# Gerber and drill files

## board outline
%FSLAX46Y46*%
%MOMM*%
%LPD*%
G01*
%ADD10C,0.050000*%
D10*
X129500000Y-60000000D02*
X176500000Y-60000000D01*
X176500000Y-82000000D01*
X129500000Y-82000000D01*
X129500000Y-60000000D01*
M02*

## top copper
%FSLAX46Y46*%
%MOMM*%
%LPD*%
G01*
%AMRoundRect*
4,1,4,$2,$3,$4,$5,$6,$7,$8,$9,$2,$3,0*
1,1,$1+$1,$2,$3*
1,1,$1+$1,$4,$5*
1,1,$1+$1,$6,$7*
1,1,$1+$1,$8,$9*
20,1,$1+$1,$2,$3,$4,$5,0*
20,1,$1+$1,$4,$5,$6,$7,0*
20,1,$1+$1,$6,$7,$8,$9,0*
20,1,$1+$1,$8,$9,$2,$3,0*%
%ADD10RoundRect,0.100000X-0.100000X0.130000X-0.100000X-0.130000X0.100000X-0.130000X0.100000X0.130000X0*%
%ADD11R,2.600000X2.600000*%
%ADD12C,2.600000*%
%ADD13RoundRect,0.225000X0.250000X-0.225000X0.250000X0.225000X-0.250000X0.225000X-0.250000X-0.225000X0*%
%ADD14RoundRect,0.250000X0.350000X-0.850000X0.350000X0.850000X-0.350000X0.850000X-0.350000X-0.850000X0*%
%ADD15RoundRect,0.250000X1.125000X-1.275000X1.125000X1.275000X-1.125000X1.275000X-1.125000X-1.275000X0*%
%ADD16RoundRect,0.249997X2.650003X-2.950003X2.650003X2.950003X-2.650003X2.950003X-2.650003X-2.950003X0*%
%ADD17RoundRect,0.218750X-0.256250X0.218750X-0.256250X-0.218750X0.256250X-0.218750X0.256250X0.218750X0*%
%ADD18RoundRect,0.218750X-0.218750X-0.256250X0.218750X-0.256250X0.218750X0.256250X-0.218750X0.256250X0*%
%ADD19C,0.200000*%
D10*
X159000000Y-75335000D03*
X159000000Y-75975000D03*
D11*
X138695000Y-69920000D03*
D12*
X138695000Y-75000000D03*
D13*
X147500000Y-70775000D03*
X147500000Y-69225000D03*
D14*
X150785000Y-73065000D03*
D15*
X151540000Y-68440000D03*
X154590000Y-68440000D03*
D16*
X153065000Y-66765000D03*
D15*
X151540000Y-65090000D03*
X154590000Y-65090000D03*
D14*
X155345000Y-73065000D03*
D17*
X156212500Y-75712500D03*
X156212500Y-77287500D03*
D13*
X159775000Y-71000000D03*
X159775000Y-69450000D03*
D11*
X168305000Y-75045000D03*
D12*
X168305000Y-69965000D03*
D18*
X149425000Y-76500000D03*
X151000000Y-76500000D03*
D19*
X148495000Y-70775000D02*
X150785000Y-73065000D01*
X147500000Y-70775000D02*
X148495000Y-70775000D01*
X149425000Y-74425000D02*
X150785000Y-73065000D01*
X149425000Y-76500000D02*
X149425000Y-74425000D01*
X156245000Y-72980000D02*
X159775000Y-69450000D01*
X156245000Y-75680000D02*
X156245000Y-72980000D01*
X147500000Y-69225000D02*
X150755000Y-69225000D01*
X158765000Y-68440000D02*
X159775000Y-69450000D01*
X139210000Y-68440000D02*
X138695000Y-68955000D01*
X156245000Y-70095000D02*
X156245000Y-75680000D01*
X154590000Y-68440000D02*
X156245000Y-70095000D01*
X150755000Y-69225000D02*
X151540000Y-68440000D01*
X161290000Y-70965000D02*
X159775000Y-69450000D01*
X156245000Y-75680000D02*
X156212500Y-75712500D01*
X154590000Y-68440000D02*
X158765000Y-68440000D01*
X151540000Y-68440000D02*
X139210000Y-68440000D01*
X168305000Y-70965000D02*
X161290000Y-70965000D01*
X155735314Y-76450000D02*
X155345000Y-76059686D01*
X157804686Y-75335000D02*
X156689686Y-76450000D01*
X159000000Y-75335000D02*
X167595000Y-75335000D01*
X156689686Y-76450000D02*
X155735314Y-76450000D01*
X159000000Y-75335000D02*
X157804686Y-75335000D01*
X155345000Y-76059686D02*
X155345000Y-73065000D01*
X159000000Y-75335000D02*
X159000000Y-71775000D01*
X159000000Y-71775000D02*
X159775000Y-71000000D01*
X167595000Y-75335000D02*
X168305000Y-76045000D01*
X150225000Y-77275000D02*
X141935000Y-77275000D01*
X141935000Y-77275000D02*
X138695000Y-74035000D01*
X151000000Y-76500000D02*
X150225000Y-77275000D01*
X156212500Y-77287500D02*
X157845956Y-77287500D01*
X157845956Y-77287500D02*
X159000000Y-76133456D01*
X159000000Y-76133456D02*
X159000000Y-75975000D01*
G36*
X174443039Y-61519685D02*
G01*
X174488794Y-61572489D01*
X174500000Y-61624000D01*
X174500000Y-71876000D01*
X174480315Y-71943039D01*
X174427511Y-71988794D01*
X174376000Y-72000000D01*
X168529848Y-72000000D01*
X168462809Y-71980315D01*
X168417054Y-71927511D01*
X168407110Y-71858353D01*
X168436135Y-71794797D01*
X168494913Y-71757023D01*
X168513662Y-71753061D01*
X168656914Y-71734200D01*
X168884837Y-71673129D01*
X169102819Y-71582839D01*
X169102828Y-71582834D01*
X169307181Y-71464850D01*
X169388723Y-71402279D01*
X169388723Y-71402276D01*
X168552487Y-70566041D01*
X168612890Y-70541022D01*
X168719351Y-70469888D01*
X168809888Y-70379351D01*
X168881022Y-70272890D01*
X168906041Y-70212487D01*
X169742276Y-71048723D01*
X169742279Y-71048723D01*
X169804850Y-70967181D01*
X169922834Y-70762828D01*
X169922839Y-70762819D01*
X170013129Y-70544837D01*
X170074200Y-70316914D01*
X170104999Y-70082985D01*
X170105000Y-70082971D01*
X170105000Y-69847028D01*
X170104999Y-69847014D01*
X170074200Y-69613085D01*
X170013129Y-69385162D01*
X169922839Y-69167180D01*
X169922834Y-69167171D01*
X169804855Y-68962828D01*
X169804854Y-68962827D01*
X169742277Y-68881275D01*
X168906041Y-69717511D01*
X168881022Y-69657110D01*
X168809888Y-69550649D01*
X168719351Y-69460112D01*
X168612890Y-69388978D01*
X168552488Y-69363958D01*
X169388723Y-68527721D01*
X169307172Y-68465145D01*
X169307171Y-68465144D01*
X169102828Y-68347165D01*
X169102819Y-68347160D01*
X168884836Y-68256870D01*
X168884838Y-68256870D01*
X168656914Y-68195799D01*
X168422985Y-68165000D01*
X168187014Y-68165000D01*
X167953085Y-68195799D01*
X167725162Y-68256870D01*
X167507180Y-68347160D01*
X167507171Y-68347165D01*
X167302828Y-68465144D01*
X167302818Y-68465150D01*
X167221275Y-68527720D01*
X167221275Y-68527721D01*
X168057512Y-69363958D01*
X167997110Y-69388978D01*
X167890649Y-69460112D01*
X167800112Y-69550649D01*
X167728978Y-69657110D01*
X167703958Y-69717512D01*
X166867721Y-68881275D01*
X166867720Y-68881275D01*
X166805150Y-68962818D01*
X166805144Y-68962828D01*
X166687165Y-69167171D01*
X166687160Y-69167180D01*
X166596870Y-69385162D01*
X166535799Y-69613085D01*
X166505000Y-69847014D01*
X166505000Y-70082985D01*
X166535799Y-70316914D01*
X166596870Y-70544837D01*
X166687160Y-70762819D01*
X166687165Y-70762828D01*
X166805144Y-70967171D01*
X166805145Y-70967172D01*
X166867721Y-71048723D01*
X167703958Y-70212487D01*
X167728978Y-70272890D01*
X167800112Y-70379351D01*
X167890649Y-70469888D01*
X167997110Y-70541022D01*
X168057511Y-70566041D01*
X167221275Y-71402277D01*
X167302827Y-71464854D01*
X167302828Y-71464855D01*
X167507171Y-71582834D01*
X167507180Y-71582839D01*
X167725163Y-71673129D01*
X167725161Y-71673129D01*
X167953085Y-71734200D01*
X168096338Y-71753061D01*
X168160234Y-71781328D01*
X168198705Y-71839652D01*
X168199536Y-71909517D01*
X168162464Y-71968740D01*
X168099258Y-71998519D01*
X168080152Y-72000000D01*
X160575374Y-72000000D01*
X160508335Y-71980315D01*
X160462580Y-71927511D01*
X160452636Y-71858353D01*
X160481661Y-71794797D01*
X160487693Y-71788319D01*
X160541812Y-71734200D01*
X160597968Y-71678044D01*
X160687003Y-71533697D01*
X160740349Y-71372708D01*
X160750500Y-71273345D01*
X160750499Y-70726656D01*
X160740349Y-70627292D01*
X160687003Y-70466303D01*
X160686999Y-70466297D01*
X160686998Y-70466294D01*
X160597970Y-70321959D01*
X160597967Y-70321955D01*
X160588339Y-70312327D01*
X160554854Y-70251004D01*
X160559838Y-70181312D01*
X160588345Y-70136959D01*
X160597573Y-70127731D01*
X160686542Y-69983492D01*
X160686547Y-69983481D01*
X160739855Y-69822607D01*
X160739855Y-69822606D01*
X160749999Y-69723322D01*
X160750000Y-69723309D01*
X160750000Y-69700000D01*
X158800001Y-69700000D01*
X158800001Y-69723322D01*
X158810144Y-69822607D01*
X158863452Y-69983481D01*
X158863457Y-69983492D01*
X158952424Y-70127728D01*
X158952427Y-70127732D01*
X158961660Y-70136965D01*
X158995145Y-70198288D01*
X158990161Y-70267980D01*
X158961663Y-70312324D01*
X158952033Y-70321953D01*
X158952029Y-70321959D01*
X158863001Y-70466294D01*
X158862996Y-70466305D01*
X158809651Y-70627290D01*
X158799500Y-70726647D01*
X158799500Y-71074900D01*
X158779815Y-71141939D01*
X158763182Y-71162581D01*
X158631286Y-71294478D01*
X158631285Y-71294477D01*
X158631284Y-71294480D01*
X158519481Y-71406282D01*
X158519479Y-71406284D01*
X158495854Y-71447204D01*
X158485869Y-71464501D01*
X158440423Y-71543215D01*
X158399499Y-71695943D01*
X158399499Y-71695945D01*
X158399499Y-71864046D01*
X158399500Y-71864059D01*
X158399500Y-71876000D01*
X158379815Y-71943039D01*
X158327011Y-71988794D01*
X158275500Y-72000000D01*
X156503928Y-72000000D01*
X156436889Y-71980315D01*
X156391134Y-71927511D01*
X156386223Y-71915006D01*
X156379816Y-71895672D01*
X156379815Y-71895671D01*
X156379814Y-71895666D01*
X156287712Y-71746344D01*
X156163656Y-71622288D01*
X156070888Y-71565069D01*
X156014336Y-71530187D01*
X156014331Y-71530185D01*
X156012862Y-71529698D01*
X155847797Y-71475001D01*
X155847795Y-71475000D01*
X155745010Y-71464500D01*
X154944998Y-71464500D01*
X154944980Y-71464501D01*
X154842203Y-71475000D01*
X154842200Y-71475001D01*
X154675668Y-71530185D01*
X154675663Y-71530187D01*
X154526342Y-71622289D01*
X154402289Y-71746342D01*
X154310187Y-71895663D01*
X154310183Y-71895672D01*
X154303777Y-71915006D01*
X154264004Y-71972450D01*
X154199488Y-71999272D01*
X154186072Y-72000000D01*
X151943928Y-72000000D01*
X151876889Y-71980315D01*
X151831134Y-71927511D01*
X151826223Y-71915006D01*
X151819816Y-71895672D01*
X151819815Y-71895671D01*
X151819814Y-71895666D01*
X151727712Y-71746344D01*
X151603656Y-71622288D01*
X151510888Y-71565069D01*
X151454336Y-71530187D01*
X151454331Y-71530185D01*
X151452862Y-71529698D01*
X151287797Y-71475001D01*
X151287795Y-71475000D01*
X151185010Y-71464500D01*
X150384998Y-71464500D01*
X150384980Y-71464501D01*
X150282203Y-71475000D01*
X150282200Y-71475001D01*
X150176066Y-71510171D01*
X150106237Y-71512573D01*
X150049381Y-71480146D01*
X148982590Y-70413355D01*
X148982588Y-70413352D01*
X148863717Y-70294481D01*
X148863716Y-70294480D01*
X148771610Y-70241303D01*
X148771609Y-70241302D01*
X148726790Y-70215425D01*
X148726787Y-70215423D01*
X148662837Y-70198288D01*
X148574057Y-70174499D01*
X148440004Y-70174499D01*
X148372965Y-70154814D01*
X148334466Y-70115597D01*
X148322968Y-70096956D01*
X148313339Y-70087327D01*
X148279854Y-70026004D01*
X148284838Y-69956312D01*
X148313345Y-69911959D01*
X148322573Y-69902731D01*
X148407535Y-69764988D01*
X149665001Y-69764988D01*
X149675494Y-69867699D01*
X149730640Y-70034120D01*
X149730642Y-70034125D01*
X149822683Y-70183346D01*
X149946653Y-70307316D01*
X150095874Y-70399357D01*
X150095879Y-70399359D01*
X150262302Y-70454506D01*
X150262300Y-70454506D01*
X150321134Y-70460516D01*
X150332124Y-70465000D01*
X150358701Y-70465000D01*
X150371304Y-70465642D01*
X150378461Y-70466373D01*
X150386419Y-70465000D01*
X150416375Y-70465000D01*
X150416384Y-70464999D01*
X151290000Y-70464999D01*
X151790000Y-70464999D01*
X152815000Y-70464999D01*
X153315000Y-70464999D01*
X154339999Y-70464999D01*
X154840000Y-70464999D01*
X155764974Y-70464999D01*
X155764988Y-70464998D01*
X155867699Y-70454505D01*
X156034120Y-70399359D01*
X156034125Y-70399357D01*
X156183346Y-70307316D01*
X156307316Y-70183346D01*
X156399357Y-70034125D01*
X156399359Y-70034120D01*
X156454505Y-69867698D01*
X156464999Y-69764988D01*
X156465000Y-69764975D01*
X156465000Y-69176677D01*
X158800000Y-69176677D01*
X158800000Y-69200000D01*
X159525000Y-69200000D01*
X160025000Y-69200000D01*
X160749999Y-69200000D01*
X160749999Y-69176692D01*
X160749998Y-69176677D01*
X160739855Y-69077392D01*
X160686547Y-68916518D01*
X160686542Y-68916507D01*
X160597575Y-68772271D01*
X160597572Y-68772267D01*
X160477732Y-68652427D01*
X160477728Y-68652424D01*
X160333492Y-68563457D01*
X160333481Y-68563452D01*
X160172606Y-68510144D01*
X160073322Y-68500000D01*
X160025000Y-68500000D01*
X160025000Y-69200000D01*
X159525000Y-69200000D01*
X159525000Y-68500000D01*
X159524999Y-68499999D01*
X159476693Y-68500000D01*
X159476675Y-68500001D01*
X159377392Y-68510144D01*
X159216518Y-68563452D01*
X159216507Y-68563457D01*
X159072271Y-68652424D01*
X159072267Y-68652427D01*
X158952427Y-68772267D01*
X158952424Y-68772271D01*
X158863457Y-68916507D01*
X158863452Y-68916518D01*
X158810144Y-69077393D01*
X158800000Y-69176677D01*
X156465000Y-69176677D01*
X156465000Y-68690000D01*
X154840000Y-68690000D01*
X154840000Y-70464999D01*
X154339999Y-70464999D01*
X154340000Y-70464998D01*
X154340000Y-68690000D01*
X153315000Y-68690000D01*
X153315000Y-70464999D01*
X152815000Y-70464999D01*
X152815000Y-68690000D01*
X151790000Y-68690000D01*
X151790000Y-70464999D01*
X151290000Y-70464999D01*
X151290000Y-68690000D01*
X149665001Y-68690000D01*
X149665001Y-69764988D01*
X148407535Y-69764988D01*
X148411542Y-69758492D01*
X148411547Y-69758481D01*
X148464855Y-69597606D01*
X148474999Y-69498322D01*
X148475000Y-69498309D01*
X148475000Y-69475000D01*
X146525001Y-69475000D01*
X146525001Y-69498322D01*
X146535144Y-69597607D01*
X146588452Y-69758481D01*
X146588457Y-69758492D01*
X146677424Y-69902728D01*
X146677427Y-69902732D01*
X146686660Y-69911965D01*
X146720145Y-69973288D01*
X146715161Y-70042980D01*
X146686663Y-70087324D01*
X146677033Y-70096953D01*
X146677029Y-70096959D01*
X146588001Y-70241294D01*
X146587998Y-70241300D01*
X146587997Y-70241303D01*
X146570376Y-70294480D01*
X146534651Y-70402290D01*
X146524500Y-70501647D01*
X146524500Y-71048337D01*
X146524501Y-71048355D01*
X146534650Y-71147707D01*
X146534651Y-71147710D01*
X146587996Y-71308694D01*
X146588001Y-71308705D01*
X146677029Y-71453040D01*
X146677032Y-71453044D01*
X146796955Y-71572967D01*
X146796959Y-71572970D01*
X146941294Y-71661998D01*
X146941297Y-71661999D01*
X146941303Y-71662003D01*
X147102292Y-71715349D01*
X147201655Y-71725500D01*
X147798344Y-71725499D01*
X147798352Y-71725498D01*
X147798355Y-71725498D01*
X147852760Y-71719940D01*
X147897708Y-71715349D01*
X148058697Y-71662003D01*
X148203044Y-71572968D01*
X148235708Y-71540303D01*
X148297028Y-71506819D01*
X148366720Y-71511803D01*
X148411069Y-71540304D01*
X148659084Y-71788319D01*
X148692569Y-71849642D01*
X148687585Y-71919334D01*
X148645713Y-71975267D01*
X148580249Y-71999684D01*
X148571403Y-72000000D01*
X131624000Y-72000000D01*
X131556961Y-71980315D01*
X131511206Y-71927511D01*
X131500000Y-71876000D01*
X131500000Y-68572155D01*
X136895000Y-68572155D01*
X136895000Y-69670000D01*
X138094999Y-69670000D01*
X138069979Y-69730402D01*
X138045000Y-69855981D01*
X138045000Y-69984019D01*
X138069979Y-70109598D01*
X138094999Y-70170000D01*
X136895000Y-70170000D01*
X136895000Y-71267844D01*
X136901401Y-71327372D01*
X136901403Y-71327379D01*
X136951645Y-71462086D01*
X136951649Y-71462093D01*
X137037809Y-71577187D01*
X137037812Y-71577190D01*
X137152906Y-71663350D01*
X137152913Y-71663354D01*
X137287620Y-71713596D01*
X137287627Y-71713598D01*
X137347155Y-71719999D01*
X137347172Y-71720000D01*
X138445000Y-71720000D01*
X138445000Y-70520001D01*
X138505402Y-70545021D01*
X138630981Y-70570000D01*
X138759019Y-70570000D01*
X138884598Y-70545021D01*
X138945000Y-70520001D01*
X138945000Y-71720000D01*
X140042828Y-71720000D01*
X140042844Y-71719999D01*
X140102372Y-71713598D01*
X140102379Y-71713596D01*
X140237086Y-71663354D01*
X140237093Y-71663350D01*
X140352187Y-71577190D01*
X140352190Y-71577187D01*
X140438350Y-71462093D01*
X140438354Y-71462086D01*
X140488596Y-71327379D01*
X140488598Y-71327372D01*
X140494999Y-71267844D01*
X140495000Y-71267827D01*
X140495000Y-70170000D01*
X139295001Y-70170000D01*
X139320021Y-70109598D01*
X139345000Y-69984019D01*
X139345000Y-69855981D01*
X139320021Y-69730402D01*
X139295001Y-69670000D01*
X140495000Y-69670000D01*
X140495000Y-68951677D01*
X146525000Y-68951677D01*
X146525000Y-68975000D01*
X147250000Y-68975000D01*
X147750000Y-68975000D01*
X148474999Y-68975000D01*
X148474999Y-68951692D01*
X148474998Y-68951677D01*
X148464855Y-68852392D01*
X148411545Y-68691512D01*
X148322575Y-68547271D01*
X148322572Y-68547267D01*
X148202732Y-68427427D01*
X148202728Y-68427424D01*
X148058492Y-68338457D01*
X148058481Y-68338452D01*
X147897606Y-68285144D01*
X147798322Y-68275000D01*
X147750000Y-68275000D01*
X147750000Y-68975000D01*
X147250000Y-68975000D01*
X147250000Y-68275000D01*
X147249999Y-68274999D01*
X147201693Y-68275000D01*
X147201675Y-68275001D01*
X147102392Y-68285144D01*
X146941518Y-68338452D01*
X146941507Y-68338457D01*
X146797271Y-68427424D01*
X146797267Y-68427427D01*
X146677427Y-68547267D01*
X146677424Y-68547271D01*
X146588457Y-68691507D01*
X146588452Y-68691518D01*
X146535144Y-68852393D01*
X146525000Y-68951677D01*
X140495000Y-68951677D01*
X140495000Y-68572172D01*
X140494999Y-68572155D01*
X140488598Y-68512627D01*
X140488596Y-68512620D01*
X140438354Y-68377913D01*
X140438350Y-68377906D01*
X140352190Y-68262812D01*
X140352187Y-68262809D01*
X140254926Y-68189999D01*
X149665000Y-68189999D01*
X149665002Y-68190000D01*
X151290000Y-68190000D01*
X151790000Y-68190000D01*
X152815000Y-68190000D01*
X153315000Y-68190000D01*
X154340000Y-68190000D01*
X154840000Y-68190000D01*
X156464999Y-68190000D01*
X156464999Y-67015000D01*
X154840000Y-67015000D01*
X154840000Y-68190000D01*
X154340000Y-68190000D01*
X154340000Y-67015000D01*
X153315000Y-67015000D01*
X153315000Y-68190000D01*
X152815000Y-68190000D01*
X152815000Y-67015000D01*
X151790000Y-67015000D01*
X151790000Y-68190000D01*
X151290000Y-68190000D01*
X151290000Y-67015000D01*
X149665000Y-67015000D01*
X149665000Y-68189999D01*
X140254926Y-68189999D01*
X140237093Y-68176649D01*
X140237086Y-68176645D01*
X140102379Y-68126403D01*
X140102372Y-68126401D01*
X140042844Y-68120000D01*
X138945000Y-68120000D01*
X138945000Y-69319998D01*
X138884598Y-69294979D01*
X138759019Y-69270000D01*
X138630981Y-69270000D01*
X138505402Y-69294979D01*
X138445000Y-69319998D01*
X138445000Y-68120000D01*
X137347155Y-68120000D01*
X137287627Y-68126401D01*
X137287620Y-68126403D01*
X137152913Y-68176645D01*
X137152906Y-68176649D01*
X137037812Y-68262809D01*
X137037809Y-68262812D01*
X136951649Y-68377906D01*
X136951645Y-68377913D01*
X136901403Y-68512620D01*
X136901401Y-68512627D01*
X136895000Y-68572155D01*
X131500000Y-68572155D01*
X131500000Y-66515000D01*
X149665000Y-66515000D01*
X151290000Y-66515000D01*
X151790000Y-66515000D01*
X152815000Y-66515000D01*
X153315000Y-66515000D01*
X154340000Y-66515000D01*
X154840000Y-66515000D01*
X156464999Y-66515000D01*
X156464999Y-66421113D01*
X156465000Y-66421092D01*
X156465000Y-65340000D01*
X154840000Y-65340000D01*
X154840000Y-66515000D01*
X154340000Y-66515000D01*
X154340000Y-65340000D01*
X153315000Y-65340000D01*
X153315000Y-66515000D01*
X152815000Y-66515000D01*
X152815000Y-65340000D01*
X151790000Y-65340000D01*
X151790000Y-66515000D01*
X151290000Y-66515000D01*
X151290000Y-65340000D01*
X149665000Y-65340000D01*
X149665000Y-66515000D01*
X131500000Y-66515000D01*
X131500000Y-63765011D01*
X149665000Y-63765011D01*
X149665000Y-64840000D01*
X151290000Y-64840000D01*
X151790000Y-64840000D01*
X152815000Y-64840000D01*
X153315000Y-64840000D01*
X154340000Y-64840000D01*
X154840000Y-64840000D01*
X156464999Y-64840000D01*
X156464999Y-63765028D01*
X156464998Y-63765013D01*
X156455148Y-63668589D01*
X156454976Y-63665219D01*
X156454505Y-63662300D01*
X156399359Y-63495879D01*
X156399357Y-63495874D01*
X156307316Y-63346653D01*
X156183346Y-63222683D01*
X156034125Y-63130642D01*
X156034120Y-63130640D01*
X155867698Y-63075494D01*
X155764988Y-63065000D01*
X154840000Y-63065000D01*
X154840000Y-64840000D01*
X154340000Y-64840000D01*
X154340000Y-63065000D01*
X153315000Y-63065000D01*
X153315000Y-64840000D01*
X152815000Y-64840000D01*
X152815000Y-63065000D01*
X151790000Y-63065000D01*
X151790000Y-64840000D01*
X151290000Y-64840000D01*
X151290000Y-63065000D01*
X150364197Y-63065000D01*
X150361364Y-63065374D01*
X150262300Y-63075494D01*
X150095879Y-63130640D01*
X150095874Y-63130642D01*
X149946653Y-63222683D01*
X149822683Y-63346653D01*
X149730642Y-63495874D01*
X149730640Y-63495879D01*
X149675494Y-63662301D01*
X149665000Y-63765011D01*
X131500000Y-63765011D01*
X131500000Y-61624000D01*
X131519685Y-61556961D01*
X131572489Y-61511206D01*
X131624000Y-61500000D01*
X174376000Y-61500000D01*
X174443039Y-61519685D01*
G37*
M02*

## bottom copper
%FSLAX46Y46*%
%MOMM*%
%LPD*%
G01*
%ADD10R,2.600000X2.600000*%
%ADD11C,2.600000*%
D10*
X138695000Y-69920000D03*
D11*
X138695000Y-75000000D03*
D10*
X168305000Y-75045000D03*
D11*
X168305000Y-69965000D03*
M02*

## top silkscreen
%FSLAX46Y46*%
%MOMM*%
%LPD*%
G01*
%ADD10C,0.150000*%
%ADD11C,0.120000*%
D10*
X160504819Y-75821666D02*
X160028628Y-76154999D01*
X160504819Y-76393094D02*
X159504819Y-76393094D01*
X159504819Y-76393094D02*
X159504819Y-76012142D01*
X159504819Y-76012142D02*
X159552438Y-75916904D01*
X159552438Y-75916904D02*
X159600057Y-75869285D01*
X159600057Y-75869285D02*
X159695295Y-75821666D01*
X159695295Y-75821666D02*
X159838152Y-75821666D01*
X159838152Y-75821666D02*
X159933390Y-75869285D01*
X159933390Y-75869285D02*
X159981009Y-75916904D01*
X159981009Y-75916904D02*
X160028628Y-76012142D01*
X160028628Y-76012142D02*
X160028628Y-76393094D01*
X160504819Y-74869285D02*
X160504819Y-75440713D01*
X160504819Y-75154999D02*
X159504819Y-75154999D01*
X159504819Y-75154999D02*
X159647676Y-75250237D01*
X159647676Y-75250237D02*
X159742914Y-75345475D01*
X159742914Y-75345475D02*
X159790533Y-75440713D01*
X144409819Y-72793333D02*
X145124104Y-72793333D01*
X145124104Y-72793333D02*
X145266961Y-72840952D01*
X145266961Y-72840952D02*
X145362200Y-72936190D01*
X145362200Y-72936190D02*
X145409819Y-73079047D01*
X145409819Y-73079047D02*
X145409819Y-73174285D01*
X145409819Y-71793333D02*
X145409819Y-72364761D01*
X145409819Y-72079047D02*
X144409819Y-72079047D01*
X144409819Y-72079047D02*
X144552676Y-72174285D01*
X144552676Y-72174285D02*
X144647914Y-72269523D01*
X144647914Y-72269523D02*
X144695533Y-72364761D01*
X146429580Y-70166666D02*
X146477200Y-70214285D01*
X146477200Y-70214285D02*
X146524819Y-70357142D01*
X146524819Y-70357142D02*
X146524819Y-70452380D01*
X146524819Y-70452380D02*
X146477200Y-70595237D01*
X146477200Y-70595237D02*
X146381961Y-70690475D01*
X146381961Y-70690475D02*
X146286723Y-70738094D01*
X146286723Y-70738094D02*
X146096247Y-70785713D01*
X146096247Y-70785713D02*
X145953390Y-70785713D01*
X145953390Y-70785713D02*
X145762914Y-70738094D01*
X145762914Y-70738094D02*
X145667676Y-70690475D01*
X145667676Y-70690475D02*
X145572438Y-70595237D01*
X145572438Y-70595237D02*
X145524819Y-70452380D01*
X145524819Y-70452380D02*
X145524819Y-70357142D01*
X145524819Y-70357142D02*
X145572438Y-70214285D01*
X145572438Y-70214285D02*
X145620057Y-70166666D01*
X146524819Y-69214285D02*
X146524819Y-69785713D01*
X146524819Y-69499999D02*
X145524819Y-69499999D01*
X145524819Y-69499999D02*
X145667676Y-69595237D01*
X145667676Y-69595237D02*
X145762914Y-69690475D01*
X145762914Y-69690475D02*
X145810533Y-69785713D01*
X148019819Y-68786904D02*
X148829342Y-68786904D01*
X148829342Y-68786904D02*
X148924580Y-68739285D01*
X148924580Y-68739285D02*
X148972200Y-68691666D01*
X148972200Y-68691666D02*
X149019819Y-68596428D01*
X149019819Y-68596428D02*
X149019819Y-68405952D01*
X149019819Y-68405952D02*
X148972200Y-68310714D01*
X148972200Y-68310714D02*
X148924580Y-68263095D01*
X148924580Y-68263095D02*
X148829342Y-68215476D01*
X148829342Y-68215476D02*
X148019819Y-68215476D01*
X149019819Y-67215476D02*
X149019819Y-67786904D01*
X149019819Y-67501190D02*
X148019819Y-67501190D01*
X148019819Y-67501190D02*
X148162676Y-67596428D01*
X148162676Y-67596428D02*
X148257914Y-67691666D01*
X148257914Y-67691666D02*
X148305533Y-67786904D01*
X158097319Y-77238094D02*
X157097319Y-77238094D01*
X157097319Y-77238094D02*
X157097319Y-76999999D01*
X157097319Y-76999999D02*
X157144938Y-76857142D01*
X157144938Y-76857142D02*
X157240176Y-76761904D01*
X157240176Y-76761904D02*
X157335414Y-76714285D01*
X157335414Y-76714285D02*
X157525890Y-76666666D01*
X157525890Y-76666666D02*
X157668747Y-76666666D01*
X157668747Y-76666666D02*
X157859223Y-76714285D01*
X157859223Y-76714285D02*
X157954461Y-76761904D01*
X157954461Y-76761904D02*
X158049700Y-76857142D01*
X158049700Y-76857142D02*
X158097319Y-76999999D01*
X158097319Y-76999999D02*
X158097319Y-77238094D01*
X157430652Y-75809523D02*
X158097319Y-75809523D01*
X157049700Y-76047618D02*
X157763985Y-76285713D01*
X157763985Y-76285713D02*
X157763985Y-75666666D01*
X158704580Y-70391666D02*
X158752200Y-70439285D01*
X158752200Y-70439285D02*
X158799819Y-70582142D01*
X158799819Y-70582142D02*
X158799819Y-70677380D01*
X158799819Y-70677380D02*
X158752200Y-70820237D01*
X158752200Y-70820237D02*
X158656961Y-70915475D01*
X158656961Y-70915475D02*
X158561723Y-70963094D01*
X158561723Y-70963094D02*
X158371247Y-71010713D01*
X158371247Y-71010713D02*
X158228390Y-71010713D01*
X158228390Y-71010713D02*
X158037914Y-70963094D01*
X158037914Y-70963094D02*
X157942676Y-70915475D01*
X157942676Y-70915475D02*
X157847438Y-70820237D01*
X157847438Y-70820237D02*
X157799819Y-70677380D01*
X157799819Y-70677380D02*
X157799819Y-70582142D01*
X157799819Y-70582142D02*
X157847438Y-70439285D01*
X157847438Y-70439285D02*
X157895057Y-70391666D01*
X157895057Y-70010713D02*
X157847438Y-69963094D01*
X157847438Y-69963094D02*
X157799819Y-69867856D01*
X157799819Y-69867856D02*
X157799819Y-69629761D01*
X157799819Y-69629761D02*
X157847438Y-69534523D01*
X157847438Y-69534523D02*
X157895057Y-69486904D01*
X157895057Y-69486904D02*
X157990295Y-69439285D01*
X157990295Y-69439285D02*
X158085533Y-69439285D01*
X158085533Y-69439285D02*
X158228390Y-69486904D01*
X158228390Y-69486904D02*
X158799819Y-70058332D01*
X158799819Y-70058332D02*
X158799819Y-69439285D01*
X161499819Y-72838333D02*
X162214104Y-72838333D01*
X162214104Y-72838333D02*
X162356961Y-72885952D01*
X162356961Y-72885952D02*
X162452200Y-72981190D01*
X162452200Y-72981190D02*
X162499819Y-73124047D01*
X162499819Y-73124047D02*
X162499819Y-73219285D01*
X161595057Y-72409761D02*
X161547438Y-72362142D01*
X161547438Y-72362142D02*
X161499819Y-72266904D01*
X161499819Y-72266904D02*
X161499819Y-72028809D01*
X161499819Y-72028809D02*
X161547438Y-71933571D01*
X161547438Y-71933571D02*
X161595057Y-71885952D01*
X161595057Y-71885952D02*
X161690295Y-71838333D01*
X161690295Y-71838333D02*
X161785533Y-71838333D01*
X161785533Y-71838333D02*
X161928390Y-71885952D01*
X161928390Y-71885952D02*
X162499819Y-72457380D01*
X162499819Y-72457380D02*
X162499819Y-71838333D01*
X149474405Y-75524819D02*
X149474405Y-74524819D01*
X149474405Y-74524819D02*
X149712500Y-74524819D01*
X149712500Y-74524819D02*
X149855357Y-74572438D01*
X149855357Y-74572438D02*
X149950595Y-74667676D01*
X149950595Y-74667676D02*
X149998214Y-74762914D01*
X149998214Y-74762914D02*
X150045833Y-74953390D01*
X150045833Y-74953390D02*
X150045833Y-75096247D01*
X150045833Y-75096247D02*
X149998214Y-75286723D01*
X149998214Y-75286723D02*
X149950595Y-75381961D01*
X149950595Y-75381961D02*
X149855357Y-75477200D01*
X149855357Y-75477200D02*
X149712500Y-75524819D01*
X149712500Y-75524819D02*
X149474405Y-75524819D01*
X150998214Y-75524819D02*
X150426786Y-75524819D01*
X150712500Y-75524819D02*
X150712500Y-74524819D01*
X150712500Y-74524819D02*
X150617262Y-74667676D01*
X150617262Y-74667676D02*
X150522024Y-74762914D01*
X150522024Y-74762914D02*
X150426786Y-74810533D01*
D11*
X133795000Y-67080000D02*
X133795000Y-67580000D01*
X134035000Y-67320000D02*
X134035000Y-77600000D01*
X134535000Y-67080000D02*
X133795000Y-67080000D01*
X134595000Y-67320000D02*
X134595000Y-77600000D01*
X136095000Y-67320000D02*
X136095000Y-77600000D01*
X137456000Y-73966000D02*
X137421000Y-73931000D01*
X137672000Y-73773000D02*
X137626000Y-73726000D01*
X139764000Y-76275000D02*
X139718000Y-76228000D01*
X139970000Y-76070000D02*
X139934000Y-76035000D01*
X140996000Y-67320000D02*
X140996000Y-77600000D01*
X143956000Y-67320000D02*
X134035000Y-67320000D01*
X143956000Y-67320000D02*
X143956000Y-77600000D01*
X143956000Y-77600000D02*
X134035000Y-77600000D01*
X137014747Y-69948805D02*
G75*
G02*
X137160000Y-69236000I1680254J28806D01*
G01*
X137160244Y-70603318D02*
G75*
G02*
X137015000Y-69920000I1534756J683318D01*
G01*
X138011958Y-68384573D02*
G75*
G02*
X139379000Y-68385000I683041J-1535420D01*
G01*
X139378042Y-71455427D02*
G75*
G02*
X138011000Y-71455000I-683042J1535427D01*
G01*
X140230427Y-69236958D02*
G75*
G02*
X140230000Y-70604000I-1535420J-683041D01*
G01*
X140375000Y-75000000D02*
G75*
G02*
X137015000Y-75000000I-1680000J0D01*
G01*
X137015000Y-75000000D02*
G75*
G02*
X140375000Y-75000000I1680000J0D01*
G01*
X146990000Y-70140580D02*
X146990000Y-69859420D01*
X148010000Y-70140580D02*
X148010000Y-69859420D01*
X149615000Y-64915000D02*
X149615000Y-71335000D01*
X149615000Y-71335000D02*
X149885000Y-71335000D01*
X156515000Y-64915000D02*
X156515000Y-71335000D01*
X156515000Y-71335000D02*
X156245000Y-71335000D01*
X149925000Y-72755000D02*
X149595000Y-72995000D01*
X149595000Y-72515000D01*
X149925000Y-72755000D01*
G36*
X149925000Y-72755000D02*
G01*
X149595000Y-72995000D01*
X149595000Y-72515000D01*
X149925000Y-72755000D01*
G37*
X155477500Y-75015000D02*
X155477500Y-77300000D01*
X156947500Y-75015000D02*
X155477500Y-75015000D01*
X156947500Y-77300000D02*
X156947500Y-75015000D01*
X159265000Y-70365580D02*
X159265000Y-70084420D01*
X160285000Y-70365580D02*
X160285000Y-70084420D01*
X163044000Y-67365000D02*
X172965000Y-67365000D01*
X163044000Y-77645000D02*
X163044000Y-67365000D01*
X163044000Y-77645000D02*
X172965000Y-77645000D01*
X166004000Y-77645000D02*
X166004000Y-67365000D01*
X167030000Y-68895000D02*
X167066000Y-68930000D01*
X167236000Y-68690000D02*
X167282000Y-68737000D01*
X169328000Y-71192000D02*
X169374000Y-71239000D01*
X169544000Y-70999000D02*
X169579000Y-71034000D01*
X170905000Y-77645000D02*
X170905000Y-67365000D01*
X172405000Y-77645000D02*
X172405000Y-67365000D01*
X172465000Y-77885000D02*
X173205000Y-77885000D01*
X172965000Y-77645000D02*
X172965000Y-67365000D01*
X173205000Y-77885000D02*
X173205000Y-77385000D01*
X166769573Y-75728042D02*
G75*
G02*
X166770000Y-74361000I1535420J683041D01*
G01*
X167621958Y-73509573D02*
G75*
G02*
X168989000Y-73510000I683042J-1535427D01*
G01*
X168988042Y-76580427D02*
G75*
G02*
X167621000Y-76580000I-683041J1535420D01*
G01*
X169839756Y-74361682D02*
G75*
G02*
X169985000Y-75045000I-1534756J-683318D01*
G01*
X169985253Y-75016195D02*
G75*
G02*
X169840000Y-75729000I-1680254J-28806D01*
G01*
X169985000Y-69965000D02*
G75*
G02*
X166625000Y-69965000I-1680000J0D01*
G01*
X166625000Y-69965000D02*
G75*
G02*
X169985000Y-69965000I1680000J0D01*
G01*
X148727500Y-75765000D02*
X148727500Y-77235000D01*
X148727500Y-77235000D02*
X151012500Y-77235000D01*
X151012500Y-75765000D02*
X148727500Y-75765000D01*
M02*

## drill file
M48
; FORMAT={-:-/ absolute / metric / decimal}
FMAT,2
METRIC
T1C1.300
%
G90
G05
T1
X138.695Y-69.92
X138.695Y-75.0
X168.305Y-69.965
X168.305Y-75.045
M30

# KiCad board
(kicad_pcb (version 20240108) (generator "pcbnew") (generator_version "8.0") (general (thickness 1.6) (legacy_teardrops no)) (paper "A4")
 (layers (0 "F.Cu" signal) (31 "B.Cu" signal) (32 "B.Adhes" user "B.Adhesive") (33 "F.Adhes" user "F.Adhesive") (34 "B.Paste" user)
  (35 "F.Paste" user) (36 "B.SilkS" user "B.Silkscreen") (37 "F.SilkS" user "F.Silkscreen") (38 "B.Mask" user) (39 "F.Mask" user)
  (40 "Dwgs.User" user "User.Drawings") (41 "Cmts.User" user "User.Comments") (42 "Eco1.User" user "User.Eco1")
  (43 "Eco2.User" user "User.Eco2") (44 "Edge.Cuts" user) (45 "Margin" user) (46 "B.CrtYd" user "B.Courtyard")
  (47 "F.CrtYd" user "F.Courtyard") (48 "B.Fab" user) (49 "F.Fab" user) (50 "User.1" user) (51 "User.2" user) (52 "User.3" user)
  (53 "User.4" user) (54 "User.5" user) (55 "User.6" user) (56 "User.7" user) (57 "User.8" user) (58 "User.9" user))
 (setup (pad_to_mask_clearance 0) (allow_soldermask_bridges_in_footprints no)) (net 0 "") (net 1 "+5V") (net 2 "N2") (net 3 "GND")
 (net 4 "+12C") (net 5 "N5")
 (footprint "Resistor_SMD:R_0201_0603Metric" (layer "F.Cu") (at 159 75.655 -90)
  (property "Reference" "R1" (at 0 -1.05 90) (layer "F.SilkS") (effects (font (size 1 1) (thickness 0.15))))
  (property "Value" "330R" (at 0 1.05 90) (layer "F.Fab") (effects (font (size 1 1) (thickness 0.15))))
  (pad "" smd roundrect (at -0.345 0 270) (size 0.318 0.36) (layers "F.Paste") (roundrect_rratio 0.25))
  (pad "" smd roundrect (at 0.345 0 270) (size 0.318 0.36) (layers "F.Paste") (roundrect_rratio 0.25))
  (pad "1" smd roundrect (at -0.32 0 270) (size 0.46 0.4) (layers "F.Cu" "F.Mask") (roundrect_rratio 0.25) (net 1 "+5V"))
  (pad "2" smd roundrect (at 0.32 0 270) (size 0.46 0.4) (layers "F.Cu" "F.Mask") (roundrect_rratio 0.25) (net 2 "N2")))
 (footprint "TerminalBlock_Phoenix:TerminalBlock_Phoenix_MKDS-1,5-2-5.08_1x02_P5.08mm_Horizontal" (layer "F.Cu") (at 138.695 69.92 -90)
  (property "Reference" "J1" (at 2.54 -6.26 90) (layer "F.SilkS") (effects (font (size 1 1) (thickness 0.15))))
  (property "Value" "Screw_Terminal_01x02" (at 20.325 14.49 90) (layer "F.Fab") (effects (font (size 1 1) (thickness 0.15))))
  (fp_line (start -2.84 4.9) (end -2.34 4.9) (stroke (width 0.12) (type solid)) (layer "F.SilkS"))
  (fp_line (start -2.6 4.66) (end 7.68 4.66) (stroke (width 0.12) (type solid)) (layer "F.SilkS"))
  (fp_line (start -2.84 4.16) (end -2.84 4.9) (stroke (width 0.12) (type solid)) (layer "F.SilkS"))
  (fp_line (start -2.6 4.1) (end 7.68 4.1) (stroke (width 0.12) (type solid)) (layer "F.SilkS"))
  (fp_line (start -2.6 2.6) (end 7.68 2.6) (stroke (width 0.12) (type solid)) (layer "F.SilkS"))
  (fp_line (start 4.046 1.239) (end 4.011 1.274) (stroke (width 0.12) (type solid)) (layer "F.SilkS"))
  (fp_line (start 3.853 1.023) (end 3.806 1.069) (stroke (width 0.12) (type solid)) (layer "F.SilkS"))
  (fp_line (start 6.355 -1.069) (end 6.308 -1.023) (stroke (width 0.12) (type solid)) (layer "F.SilkS"))
  (fp_line (start 6.15 -1.275) (end 6.115 -1.239) (stroke (width 0.12) (type solid)) (layer "F.SilkS"))
  (fp_line (start -2.6 -2.301) (end 7.68 -2.301) (stroke (width 0.12) (type solid)) (layer "F.SilkS"))
  (fp_line (start -2.6 -5.261) (end -2.6 4.66) (stroke (width 0.12) (type solid)) (layer "F.SilkS"))
  (fp_line (start -2.6 -5.261) (end 7.68 -5.261) (stroke (width 0.12) (type solid)) (layer "F.SilkS"))
  (fp_line (start 7.68 -5.261) (end 7.68 4.66) (stroke (width 0.12) (type solid)) (layer "F.SilkS"))
  (fp_arc (start 0.028805 1.680253) (mid -0.335551 1.646659) (end -0.684 1.535) (stroke (width 0.12) (type solid)) (layer "F.SilkS"))
  (fp_arc (start 0.683318 1.534756) (mid 0.349292 1.643288) (end 0 1.68) (stroke (width 0.12) (type solid)) (layer "F.SilkS"))
  (fp_arc (start -1.535427 0.683042) (mid -1.680501 -0.000524) (end -1.535 -0.684) (stroke (width 0.12) (type solid)) (layer "F.SilkS"))
  (fp_arc (start 1.535427 -0.683042) (mid 1.680501 0.000524) (end 1.535 0.684) (stroke (width 0.12) (type solid)) (layer "F.SilkS"))
  (fp_arc (start -0.683042 -1.535427) (mid 0.000524 -1.680501) (end 0.684 -1.535) (stroke (width 0.12) (type solid)) (layer "F.SilkS"))
  (fp_circle (center 5.08 0) (end 6.76 0) (stroke (width 0.12) (type solid)) (fill none) (layer "F.SilkS"))
  (pad "1" thru_hole rect (at 0 0 270) (size 2.6 2.6) (drill 1.3) (layers "*.Cu" "*.Mask") (remove_unused_layers no) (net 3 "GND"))
  (pad "2" thru_hole circle (at 5.08 0 270) (size 2.6 2.6) (drill 1.3) (layers "*.Cu" "*.Mask") (remove_unused_layers no) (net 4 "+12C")))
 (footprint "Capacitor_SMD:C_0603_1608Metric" (layer "F.Cu") (at 147.5 70 90)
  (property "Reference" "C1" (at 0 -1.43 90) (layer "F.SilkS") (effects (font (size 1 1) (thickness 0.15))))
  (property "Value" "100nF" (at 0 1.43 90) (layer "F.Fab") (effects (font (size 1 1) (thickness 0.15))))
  (fp_line (start -0.14058 -0.51) (end 0.14058 -0.51) (stroke (width 0.12) (type solid)) (layer "F.SilkS"))
  (fp_line (start -0.14058 0.51) (end 0.14058 0.51) (stroke (width 0.12) (type solid)) (layer "F.SilkS"))
  (pad "1" smd roundrect (at -0.775 0 90) (size 0.9 0.95) (layers "F.Cu" "F.Paste" "F.Mask") (roundrect_rratio 0.25) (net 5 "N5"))
  (pad "2" smd roundrect (at 0.775 0 90) (size 0.9 0.95) (layers "F.Cu" "F.Paste" "F.Mask") (roundrect_rratio 0.25) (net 3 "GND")))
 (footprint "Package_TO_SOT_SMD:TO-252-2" (layer "F.Cu") (at 153.065 68.025 90)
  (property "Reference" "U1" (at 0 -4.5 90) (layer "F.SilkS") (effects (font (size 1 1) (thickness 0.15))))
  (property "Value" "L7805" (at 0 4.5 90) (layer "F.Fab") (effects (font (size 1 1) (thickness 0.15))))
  (fp_line (start 3.11 -3.45) (end -3.31 -3.45) (stroke (width 0.12) (type solid)) (layer "F.SilkS"))
  (fp_line (start -3.31 -3.45) (end -3.31 -3.18) (stroke (width 0.12) (type solid)) (layer "F.SilkS"))
  (fp_line (start 3.11 3.45) (end -3.31 3.45) (stroke (width 0.12) (type solid)) (layer "F.SilkS"))
  (fp_line (start -3.31 3.45) (end -3.31 3.18) (stroke (width 0.12) (type solid)) (layer "F.SilkS"))
  (fp_poly
   (pts (xy -4.73 -3.14) (xy -4.97 -3.47) (xy -4.49 -3.47) (xy -4.73 -3.14)) (stroke (width 0.12) (type solid)) (fill solid)
   (layer "F.SilkS"))
  (pad "1" smd roundrect (at -5.04 -2.28 90) (size 2.2 1.2) (layers "F.Cu" "F.Paste" "F.Mask") (roundrect_rratio 0.208333) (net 5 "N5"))
  (pad "2" smd roundrect (at -0.415 -1.525 90) (size 3.05 2.75) (layers "F.Cu" "F.Paste") (roundrect_rratio 0.090909) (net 3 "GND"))
  (pad "2" smd roundrect (at -0.415 1.525 90) (size 3.05 2.75) (layers "F.Cu" "F.Paste") (roundrect_rratio 0.090909) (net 3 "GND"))
  (pad "2" smd roundrect (at 1.26 0 90) (size 6.4 5.8) (layers "F.Cu" "F.Mask") (roundrect_rratio 0.043103) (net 3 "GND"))
  (pad "2" smd roundrect (at 2.935 -1.525 90) (size 3.05 2.75) (layers "F.Cu" "F.Paste") (roundrect_rratio 0.090909) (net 3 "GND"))
  (pad "2" smd roundrect (at 2.935 1.525 90) (size 3.05 2.75) (layers "F.Cu" "F.Paste") (roundrect_rratio 0.090909) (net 3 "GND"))
  (pad "3" smd roundrect (at -5.04 2.28 90) (size 2.2 1.2) (layers "F.Cu" "F.Paste" "F.Mask") (roundrect_rratio 0.208333) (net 1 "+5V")))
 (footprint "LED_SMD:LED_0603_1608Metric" (layer "F.Cu") (at 156.2125 76.5 -90)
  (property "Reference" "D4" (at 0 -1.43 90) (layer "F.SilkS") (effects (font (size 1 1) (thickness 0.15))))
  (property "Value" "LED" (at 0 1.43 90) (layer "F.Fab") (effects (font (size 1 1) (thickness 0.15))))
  (fp_line (start -1.485 0.735) (end 0.8 0.735) (stroke (width 0.12) (type solid)) (layer "F.SilkS"))
  (fp_line (start -1.485 -0.735) (end -1.485 0.735) (stroke (width 0.12) (type solid)) (layer "F.SilkS"))
  (fp_line (start 0.8 -0.735) (end -1.485 -0.735) (stroke (width 0.12) (type solid)) (layer "F.SilkS"))
  (pad "1" smd roundrect (at -0.7875 0 270) (size 0.875 0.95) (layers "F.Cu" "F.Paste" "F.Mask") (roundrect_rratio 0.25) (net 3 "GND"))
  (pad "2" smd roundrect (at 0.7875 0 270) (size 0.875 0.95) (layers "F.Cu" "F.Paste" "F.Mask") (roundrect_rratio 0.25) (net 2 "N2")))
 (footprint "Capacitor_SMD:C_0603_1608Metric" (layer "F.Cu") (at 159.775 70.225 90)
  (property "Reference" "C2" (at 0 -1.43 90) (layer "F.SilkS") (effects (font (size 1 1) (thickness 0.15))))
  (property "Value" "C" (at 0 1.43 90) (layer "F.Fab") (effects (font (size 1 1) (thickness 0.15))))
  (fp_line (start -0.14058 -0.51) (end 0.14058 -0.51) (stroke (width 0.12) (type solid)) (layer "F.SilkS"))
  (fp_line (start -0.14058 0.51) (end 0.14058 0.51) (stroke (width 0.12) (type solid)) (layer "F.SilkS"))
  (pad "1" smd roundrect (at -0.775 0 90) (size 0.9 0.95) (layers "F.Cu" "F.Paste" "F.Mask") (roundrect_rratio 0.25) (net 1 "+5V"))
  (pad "2" smd roundrect (at 0.775 0 90) (size 0.9 0.95) (layers "F.Cu" "F.Paste" "F.Mask") (roundrect_rratio 0.25) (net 3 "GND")))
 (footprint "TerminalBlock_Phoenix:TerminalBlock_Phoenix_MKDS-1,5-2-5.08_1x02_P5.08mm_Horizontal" (layer "F.Cu") (at 168.305 75.045 90)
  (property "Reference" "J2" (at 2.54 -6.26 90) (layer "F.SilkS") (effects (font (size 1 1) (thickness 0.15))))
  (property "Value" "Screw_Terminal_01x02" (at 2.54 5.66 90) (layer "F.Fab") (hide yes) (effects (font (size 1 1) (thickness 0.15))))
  (fp_line (start 7.68 -5.261) (end 7.68 4.66) (stroke (width 0.12) (type solid)) (layer "F.SilkS"))
  (fp_line (start -2.6 -5.261) (end 7.68 -5.261) (stroke (width 0.12) (type solid)) (layer "F.SilkS"))
  (fp_line (start -2.6 -5.261) (end -2.6 4.66) (stroke (width 0.12) (type solid)) (layer "F.SilkS"))
  (fp_line (start -2.6 -2.301) (end 7.68 -2.301) (stroke (width 0.12) (type solid)) (layer "F.SilkS"))
  (fp_line (start 6.15 -1.275) (end 6.115 -1.239) (stroke (width 0.12) (type solid)) (layer "F.SilkS"))
  (fp_line (start 6.355 -1.069) (end 6.308 -1.023) (stroke (width 0.12) (type solid)) (layer "F.SilkS"))
  (fp_line (start 3.853 1.023) (end 3.806 1.069) (stroke (width 0.12) (type solid)) (layer "F.SilkS"))
  (fp_line (start 4.046 1.239) (end 4.011 1.274) (stroke (width 0.12) (type solid)) (layer "F.SilkS"))
  (fp_line (start -2.6 2.6) (end 7.68 2.6) (stroke (width 0.12) (type solid)) (layer "F.SilkS"))
  (fp_line (start -2.6 4.1) (end 7.68 4.1) (stroke (width 0.12) (type solid)) (layer "F.SilkS"))
  (fp_line (start -2.84 4.16) (end -2.84 4.9) (stroke (width 0.12) (type solid)) (layer "F.SilkS"))
  (fp_line (start -2.6 4.66) (end 7.68 4.66) (stroke (width 0.12) (type solid)) (layer "F.SilkS"))
  (fp_line (start -2.84 4.9) (end -2.34 4.9) (stroke (width 0.12) (type solid)) (layer "F.SilkS"))
  (fp_arc (start -0.683042 -1.535427) (mid 0.000524 -1.680501) (end 0.684 -1.535) (stroke (width 0.12) (type solid)) (layer "F.SilkS"))
  (fp_arc (start 1.535427 -0.683042) (mid 1.680501 0.000524) (end 1.535 0.684) (stroke (width 0.12) (type solid)) (layer "F.SilkS"))
  (fp_arc (start -1.535427 0.683042) (mid -1.680501 -0.000524) (end -1.535 -0.684) (stroke (width 0.12) (type solid)) (layer "F.SilkS"))
  (fp_arc (start 0.683318 1.534756) (mid 0.349292 1.643288) (end 0 1.68) (stroke (width 0.12) (type solid)) (layer "F.SilkS"))
  (fp_arc (start 0.028805 1.680253) (mid -0.335551 1.646659) (end -0.684 1.535) (stroke (width 0.12) (type solid)) (layer "F.SilkS"))
  (fp_circle (center 5.08 0) (end 6.76 0) (stroke (width 0.12) (type solid)) (fill none) (layer "F.SilkS"))
  (pad "1" thru_hole rect (at 0 0 90) (size 2.6 2.6) (drill 1.3) (layers "*.Cu" "*.Mask") (remove_unused_layers no) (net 1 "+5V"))
  (pad "2" thru_hole circle (at 5.08 0 90) (size 2.6 2.6) (drill 1.3) (layers "*.Cu" "*.Mask") (remove_unused_layers no) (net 3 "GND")))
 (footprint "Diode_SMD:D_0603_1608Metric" (layer "F.Cu") (at 150.2125 76.5)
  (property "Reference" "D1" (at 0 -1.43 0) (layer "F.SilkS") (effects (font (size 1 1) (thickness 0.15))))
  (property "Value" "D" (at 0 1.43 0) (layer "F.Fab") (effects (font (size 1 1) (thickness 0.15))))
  (fp_line (start -1.485 -0.735) (end -1.485 0.735) (stroke (width 0.12) (type solid)) (layer "F.SilkS"))
  (fp_line (start -1.485 0.735) (end 0.8 0.735) (stroke (width 0.12) (type solid)) (layer "F.SilkS"))
  (fp_line (start 0.8 -0.735) (end -1.485 -0.735) (stroke (width 0.12) (type solid)) (layer "F.SilkS"))
  (pad "1" smd roundrect (at -0.7875 0) (size 0.875 0.95) (layers "F.Cu" "F.Paste" "F.Mask") (roundrect_rratio 0.25) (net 5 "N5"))
  (pad "2" smd roundrect (at 0.7875 0) (size 0.875 0.95) (layers "F.Cu" "F.Paste" "F.Mask") (roundrect_rratio 0.25) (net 4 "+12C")))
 (gr_rect (start 129.5 60) (end 176.5 82) (stroke (width 0.05) (type default)) (fill none) (layer "Edge.Cuts"))
 (segment (start 148.495 70.775) (end 150.785 73.065) (width 0.2) (layer "F.Cu") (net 5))
 (segment (start 147.5 70.775) (end 148.495 70.775) (width 0.2) (layer "F.Cu") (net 5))
 (segment (start 149.425 74.425) (end 150.785 73.065) (width 0.2) (layer "F.Cu") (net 5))
 (segment (start 149.425 76.5) (end 149.425 74.425) (width 0.2) (layer "F.Cu") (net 5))
 (segment (start 156.245 72.98) (end 159.775 69.45) (width 0.2) (layer "F.Cu") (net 3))
 (segment (start 156.245 75.68) (end 156.245 72.98) (width 0.2) (layer "F.Cu") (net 3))
 (segment (start 147.5 69.225) (end 150.755 69.225) (width 0.2) (layer "F.Cu") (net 3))
 (segment (start 158.765 68.44) (end 159.775 69.45) (width 0.2) (layer "F.Cu") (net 3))
 (segment (start 139.21 68.44) (end 138.695 68.955) (width 0.2) (layer "F.Cu") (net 3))
 (segment (start 156.245 70.095) (end 156.245 75.68) (width 0.2) (layer "F.Cu") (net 3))
 (segment (start 154.59 68.44) (end 156.245 70.095) (width 0.2) (layer "F.Cu") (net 3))
 (segment (start 150.755 69.225) (end 151.54 68.44) (width 0.2) (layer "F.Cu") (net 3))
 (segment (start 161.29 70.965) (end 159.775 69.45) (width 0.2) (layer "F.Cu") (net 3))
 (segment (start 156.245 75.68) (end 156.2125 75.7125) (width 0.2) (layer "F.Cu") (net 3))
 (segment (start 154.59 68.44) (end 158.765 68.44) (width 0.2) (layer "F.Cu") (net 3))
 (segment (start 151.54 68.44) (end 139.21 68.44) (width 0.2) (layer "F.Cu") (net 3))
 (segment (start 168.305 70.965) (end 161.29 70.965) (width 0.2) (layer "F.Cu") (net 3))
 (segment (start 155.735314 76.45) (end 155.345 76.059686) (width 0.2) (layer "F.Cu") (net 1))
 (segment (start 157.804686 75.335) (end 156.689686 76.45) (width 0.2) (layer "F.Cu") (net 1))
 (segment (start 159 75.335) (end 167.595 75.335) (width 0.2) (layer "F.Cu") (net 1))
 (segment (start 156.689686 76.45) (end 155.735314 76.45) (width 0.2) (layer "F.Cu") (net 1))
 (segment (start 159 75.335) (end 157.804686 75.335) (width 0.2) (layer "F.Cu") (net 1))
 (segment (start 155.345 76.059686) (end 155.345 73.065) (width 0.2) (layer "F.Cu") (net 1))
 (segment (start 159 75.335) (end 159 71.775) (width 0.2) (layer "F.Cu") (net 1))
 (segment (start 159 71.775) (end 159.775 71) (width 0.2) (layer "F.Cu") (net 1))
 (segment (start 167.595 75.335) (end 168.305 76.045) (width 0.2) (layer "F.Cu") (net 1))
 (segment (start 150.225 77.275) (end 141.935 77.275) (width 0.2) (layer "F.Cu") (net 4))
 (segment (start 141.935 77.275) (end 138.695 74.035) (width 0.2) (layer "F.Cu") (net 4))
 (segment (start 151 76.5) (end 150.225 77.275) (width 0.2) (layer "F.Cu") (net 4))
 (segment (start 156.2125 77.2875) (end 157.845956 77.2875) (width 0.2) (layer "F.Cu") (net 2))
 (segment (start 157.845956 77.2875) (end 159 76.133456) (width 0.2) (layer "F.Cu") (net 2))
 (segment (start 159 76.133456) (end 159 75.975) (width 0.2) (layer "F.Cu") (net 2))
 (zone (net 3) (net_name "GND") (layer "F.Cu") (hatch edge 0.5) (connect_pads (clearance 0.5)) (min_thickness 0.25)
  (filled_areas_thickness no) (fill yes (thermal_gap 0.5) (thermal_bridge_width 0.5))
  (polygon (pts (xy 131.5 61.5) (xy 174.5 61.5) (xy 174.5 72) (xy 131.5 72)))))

